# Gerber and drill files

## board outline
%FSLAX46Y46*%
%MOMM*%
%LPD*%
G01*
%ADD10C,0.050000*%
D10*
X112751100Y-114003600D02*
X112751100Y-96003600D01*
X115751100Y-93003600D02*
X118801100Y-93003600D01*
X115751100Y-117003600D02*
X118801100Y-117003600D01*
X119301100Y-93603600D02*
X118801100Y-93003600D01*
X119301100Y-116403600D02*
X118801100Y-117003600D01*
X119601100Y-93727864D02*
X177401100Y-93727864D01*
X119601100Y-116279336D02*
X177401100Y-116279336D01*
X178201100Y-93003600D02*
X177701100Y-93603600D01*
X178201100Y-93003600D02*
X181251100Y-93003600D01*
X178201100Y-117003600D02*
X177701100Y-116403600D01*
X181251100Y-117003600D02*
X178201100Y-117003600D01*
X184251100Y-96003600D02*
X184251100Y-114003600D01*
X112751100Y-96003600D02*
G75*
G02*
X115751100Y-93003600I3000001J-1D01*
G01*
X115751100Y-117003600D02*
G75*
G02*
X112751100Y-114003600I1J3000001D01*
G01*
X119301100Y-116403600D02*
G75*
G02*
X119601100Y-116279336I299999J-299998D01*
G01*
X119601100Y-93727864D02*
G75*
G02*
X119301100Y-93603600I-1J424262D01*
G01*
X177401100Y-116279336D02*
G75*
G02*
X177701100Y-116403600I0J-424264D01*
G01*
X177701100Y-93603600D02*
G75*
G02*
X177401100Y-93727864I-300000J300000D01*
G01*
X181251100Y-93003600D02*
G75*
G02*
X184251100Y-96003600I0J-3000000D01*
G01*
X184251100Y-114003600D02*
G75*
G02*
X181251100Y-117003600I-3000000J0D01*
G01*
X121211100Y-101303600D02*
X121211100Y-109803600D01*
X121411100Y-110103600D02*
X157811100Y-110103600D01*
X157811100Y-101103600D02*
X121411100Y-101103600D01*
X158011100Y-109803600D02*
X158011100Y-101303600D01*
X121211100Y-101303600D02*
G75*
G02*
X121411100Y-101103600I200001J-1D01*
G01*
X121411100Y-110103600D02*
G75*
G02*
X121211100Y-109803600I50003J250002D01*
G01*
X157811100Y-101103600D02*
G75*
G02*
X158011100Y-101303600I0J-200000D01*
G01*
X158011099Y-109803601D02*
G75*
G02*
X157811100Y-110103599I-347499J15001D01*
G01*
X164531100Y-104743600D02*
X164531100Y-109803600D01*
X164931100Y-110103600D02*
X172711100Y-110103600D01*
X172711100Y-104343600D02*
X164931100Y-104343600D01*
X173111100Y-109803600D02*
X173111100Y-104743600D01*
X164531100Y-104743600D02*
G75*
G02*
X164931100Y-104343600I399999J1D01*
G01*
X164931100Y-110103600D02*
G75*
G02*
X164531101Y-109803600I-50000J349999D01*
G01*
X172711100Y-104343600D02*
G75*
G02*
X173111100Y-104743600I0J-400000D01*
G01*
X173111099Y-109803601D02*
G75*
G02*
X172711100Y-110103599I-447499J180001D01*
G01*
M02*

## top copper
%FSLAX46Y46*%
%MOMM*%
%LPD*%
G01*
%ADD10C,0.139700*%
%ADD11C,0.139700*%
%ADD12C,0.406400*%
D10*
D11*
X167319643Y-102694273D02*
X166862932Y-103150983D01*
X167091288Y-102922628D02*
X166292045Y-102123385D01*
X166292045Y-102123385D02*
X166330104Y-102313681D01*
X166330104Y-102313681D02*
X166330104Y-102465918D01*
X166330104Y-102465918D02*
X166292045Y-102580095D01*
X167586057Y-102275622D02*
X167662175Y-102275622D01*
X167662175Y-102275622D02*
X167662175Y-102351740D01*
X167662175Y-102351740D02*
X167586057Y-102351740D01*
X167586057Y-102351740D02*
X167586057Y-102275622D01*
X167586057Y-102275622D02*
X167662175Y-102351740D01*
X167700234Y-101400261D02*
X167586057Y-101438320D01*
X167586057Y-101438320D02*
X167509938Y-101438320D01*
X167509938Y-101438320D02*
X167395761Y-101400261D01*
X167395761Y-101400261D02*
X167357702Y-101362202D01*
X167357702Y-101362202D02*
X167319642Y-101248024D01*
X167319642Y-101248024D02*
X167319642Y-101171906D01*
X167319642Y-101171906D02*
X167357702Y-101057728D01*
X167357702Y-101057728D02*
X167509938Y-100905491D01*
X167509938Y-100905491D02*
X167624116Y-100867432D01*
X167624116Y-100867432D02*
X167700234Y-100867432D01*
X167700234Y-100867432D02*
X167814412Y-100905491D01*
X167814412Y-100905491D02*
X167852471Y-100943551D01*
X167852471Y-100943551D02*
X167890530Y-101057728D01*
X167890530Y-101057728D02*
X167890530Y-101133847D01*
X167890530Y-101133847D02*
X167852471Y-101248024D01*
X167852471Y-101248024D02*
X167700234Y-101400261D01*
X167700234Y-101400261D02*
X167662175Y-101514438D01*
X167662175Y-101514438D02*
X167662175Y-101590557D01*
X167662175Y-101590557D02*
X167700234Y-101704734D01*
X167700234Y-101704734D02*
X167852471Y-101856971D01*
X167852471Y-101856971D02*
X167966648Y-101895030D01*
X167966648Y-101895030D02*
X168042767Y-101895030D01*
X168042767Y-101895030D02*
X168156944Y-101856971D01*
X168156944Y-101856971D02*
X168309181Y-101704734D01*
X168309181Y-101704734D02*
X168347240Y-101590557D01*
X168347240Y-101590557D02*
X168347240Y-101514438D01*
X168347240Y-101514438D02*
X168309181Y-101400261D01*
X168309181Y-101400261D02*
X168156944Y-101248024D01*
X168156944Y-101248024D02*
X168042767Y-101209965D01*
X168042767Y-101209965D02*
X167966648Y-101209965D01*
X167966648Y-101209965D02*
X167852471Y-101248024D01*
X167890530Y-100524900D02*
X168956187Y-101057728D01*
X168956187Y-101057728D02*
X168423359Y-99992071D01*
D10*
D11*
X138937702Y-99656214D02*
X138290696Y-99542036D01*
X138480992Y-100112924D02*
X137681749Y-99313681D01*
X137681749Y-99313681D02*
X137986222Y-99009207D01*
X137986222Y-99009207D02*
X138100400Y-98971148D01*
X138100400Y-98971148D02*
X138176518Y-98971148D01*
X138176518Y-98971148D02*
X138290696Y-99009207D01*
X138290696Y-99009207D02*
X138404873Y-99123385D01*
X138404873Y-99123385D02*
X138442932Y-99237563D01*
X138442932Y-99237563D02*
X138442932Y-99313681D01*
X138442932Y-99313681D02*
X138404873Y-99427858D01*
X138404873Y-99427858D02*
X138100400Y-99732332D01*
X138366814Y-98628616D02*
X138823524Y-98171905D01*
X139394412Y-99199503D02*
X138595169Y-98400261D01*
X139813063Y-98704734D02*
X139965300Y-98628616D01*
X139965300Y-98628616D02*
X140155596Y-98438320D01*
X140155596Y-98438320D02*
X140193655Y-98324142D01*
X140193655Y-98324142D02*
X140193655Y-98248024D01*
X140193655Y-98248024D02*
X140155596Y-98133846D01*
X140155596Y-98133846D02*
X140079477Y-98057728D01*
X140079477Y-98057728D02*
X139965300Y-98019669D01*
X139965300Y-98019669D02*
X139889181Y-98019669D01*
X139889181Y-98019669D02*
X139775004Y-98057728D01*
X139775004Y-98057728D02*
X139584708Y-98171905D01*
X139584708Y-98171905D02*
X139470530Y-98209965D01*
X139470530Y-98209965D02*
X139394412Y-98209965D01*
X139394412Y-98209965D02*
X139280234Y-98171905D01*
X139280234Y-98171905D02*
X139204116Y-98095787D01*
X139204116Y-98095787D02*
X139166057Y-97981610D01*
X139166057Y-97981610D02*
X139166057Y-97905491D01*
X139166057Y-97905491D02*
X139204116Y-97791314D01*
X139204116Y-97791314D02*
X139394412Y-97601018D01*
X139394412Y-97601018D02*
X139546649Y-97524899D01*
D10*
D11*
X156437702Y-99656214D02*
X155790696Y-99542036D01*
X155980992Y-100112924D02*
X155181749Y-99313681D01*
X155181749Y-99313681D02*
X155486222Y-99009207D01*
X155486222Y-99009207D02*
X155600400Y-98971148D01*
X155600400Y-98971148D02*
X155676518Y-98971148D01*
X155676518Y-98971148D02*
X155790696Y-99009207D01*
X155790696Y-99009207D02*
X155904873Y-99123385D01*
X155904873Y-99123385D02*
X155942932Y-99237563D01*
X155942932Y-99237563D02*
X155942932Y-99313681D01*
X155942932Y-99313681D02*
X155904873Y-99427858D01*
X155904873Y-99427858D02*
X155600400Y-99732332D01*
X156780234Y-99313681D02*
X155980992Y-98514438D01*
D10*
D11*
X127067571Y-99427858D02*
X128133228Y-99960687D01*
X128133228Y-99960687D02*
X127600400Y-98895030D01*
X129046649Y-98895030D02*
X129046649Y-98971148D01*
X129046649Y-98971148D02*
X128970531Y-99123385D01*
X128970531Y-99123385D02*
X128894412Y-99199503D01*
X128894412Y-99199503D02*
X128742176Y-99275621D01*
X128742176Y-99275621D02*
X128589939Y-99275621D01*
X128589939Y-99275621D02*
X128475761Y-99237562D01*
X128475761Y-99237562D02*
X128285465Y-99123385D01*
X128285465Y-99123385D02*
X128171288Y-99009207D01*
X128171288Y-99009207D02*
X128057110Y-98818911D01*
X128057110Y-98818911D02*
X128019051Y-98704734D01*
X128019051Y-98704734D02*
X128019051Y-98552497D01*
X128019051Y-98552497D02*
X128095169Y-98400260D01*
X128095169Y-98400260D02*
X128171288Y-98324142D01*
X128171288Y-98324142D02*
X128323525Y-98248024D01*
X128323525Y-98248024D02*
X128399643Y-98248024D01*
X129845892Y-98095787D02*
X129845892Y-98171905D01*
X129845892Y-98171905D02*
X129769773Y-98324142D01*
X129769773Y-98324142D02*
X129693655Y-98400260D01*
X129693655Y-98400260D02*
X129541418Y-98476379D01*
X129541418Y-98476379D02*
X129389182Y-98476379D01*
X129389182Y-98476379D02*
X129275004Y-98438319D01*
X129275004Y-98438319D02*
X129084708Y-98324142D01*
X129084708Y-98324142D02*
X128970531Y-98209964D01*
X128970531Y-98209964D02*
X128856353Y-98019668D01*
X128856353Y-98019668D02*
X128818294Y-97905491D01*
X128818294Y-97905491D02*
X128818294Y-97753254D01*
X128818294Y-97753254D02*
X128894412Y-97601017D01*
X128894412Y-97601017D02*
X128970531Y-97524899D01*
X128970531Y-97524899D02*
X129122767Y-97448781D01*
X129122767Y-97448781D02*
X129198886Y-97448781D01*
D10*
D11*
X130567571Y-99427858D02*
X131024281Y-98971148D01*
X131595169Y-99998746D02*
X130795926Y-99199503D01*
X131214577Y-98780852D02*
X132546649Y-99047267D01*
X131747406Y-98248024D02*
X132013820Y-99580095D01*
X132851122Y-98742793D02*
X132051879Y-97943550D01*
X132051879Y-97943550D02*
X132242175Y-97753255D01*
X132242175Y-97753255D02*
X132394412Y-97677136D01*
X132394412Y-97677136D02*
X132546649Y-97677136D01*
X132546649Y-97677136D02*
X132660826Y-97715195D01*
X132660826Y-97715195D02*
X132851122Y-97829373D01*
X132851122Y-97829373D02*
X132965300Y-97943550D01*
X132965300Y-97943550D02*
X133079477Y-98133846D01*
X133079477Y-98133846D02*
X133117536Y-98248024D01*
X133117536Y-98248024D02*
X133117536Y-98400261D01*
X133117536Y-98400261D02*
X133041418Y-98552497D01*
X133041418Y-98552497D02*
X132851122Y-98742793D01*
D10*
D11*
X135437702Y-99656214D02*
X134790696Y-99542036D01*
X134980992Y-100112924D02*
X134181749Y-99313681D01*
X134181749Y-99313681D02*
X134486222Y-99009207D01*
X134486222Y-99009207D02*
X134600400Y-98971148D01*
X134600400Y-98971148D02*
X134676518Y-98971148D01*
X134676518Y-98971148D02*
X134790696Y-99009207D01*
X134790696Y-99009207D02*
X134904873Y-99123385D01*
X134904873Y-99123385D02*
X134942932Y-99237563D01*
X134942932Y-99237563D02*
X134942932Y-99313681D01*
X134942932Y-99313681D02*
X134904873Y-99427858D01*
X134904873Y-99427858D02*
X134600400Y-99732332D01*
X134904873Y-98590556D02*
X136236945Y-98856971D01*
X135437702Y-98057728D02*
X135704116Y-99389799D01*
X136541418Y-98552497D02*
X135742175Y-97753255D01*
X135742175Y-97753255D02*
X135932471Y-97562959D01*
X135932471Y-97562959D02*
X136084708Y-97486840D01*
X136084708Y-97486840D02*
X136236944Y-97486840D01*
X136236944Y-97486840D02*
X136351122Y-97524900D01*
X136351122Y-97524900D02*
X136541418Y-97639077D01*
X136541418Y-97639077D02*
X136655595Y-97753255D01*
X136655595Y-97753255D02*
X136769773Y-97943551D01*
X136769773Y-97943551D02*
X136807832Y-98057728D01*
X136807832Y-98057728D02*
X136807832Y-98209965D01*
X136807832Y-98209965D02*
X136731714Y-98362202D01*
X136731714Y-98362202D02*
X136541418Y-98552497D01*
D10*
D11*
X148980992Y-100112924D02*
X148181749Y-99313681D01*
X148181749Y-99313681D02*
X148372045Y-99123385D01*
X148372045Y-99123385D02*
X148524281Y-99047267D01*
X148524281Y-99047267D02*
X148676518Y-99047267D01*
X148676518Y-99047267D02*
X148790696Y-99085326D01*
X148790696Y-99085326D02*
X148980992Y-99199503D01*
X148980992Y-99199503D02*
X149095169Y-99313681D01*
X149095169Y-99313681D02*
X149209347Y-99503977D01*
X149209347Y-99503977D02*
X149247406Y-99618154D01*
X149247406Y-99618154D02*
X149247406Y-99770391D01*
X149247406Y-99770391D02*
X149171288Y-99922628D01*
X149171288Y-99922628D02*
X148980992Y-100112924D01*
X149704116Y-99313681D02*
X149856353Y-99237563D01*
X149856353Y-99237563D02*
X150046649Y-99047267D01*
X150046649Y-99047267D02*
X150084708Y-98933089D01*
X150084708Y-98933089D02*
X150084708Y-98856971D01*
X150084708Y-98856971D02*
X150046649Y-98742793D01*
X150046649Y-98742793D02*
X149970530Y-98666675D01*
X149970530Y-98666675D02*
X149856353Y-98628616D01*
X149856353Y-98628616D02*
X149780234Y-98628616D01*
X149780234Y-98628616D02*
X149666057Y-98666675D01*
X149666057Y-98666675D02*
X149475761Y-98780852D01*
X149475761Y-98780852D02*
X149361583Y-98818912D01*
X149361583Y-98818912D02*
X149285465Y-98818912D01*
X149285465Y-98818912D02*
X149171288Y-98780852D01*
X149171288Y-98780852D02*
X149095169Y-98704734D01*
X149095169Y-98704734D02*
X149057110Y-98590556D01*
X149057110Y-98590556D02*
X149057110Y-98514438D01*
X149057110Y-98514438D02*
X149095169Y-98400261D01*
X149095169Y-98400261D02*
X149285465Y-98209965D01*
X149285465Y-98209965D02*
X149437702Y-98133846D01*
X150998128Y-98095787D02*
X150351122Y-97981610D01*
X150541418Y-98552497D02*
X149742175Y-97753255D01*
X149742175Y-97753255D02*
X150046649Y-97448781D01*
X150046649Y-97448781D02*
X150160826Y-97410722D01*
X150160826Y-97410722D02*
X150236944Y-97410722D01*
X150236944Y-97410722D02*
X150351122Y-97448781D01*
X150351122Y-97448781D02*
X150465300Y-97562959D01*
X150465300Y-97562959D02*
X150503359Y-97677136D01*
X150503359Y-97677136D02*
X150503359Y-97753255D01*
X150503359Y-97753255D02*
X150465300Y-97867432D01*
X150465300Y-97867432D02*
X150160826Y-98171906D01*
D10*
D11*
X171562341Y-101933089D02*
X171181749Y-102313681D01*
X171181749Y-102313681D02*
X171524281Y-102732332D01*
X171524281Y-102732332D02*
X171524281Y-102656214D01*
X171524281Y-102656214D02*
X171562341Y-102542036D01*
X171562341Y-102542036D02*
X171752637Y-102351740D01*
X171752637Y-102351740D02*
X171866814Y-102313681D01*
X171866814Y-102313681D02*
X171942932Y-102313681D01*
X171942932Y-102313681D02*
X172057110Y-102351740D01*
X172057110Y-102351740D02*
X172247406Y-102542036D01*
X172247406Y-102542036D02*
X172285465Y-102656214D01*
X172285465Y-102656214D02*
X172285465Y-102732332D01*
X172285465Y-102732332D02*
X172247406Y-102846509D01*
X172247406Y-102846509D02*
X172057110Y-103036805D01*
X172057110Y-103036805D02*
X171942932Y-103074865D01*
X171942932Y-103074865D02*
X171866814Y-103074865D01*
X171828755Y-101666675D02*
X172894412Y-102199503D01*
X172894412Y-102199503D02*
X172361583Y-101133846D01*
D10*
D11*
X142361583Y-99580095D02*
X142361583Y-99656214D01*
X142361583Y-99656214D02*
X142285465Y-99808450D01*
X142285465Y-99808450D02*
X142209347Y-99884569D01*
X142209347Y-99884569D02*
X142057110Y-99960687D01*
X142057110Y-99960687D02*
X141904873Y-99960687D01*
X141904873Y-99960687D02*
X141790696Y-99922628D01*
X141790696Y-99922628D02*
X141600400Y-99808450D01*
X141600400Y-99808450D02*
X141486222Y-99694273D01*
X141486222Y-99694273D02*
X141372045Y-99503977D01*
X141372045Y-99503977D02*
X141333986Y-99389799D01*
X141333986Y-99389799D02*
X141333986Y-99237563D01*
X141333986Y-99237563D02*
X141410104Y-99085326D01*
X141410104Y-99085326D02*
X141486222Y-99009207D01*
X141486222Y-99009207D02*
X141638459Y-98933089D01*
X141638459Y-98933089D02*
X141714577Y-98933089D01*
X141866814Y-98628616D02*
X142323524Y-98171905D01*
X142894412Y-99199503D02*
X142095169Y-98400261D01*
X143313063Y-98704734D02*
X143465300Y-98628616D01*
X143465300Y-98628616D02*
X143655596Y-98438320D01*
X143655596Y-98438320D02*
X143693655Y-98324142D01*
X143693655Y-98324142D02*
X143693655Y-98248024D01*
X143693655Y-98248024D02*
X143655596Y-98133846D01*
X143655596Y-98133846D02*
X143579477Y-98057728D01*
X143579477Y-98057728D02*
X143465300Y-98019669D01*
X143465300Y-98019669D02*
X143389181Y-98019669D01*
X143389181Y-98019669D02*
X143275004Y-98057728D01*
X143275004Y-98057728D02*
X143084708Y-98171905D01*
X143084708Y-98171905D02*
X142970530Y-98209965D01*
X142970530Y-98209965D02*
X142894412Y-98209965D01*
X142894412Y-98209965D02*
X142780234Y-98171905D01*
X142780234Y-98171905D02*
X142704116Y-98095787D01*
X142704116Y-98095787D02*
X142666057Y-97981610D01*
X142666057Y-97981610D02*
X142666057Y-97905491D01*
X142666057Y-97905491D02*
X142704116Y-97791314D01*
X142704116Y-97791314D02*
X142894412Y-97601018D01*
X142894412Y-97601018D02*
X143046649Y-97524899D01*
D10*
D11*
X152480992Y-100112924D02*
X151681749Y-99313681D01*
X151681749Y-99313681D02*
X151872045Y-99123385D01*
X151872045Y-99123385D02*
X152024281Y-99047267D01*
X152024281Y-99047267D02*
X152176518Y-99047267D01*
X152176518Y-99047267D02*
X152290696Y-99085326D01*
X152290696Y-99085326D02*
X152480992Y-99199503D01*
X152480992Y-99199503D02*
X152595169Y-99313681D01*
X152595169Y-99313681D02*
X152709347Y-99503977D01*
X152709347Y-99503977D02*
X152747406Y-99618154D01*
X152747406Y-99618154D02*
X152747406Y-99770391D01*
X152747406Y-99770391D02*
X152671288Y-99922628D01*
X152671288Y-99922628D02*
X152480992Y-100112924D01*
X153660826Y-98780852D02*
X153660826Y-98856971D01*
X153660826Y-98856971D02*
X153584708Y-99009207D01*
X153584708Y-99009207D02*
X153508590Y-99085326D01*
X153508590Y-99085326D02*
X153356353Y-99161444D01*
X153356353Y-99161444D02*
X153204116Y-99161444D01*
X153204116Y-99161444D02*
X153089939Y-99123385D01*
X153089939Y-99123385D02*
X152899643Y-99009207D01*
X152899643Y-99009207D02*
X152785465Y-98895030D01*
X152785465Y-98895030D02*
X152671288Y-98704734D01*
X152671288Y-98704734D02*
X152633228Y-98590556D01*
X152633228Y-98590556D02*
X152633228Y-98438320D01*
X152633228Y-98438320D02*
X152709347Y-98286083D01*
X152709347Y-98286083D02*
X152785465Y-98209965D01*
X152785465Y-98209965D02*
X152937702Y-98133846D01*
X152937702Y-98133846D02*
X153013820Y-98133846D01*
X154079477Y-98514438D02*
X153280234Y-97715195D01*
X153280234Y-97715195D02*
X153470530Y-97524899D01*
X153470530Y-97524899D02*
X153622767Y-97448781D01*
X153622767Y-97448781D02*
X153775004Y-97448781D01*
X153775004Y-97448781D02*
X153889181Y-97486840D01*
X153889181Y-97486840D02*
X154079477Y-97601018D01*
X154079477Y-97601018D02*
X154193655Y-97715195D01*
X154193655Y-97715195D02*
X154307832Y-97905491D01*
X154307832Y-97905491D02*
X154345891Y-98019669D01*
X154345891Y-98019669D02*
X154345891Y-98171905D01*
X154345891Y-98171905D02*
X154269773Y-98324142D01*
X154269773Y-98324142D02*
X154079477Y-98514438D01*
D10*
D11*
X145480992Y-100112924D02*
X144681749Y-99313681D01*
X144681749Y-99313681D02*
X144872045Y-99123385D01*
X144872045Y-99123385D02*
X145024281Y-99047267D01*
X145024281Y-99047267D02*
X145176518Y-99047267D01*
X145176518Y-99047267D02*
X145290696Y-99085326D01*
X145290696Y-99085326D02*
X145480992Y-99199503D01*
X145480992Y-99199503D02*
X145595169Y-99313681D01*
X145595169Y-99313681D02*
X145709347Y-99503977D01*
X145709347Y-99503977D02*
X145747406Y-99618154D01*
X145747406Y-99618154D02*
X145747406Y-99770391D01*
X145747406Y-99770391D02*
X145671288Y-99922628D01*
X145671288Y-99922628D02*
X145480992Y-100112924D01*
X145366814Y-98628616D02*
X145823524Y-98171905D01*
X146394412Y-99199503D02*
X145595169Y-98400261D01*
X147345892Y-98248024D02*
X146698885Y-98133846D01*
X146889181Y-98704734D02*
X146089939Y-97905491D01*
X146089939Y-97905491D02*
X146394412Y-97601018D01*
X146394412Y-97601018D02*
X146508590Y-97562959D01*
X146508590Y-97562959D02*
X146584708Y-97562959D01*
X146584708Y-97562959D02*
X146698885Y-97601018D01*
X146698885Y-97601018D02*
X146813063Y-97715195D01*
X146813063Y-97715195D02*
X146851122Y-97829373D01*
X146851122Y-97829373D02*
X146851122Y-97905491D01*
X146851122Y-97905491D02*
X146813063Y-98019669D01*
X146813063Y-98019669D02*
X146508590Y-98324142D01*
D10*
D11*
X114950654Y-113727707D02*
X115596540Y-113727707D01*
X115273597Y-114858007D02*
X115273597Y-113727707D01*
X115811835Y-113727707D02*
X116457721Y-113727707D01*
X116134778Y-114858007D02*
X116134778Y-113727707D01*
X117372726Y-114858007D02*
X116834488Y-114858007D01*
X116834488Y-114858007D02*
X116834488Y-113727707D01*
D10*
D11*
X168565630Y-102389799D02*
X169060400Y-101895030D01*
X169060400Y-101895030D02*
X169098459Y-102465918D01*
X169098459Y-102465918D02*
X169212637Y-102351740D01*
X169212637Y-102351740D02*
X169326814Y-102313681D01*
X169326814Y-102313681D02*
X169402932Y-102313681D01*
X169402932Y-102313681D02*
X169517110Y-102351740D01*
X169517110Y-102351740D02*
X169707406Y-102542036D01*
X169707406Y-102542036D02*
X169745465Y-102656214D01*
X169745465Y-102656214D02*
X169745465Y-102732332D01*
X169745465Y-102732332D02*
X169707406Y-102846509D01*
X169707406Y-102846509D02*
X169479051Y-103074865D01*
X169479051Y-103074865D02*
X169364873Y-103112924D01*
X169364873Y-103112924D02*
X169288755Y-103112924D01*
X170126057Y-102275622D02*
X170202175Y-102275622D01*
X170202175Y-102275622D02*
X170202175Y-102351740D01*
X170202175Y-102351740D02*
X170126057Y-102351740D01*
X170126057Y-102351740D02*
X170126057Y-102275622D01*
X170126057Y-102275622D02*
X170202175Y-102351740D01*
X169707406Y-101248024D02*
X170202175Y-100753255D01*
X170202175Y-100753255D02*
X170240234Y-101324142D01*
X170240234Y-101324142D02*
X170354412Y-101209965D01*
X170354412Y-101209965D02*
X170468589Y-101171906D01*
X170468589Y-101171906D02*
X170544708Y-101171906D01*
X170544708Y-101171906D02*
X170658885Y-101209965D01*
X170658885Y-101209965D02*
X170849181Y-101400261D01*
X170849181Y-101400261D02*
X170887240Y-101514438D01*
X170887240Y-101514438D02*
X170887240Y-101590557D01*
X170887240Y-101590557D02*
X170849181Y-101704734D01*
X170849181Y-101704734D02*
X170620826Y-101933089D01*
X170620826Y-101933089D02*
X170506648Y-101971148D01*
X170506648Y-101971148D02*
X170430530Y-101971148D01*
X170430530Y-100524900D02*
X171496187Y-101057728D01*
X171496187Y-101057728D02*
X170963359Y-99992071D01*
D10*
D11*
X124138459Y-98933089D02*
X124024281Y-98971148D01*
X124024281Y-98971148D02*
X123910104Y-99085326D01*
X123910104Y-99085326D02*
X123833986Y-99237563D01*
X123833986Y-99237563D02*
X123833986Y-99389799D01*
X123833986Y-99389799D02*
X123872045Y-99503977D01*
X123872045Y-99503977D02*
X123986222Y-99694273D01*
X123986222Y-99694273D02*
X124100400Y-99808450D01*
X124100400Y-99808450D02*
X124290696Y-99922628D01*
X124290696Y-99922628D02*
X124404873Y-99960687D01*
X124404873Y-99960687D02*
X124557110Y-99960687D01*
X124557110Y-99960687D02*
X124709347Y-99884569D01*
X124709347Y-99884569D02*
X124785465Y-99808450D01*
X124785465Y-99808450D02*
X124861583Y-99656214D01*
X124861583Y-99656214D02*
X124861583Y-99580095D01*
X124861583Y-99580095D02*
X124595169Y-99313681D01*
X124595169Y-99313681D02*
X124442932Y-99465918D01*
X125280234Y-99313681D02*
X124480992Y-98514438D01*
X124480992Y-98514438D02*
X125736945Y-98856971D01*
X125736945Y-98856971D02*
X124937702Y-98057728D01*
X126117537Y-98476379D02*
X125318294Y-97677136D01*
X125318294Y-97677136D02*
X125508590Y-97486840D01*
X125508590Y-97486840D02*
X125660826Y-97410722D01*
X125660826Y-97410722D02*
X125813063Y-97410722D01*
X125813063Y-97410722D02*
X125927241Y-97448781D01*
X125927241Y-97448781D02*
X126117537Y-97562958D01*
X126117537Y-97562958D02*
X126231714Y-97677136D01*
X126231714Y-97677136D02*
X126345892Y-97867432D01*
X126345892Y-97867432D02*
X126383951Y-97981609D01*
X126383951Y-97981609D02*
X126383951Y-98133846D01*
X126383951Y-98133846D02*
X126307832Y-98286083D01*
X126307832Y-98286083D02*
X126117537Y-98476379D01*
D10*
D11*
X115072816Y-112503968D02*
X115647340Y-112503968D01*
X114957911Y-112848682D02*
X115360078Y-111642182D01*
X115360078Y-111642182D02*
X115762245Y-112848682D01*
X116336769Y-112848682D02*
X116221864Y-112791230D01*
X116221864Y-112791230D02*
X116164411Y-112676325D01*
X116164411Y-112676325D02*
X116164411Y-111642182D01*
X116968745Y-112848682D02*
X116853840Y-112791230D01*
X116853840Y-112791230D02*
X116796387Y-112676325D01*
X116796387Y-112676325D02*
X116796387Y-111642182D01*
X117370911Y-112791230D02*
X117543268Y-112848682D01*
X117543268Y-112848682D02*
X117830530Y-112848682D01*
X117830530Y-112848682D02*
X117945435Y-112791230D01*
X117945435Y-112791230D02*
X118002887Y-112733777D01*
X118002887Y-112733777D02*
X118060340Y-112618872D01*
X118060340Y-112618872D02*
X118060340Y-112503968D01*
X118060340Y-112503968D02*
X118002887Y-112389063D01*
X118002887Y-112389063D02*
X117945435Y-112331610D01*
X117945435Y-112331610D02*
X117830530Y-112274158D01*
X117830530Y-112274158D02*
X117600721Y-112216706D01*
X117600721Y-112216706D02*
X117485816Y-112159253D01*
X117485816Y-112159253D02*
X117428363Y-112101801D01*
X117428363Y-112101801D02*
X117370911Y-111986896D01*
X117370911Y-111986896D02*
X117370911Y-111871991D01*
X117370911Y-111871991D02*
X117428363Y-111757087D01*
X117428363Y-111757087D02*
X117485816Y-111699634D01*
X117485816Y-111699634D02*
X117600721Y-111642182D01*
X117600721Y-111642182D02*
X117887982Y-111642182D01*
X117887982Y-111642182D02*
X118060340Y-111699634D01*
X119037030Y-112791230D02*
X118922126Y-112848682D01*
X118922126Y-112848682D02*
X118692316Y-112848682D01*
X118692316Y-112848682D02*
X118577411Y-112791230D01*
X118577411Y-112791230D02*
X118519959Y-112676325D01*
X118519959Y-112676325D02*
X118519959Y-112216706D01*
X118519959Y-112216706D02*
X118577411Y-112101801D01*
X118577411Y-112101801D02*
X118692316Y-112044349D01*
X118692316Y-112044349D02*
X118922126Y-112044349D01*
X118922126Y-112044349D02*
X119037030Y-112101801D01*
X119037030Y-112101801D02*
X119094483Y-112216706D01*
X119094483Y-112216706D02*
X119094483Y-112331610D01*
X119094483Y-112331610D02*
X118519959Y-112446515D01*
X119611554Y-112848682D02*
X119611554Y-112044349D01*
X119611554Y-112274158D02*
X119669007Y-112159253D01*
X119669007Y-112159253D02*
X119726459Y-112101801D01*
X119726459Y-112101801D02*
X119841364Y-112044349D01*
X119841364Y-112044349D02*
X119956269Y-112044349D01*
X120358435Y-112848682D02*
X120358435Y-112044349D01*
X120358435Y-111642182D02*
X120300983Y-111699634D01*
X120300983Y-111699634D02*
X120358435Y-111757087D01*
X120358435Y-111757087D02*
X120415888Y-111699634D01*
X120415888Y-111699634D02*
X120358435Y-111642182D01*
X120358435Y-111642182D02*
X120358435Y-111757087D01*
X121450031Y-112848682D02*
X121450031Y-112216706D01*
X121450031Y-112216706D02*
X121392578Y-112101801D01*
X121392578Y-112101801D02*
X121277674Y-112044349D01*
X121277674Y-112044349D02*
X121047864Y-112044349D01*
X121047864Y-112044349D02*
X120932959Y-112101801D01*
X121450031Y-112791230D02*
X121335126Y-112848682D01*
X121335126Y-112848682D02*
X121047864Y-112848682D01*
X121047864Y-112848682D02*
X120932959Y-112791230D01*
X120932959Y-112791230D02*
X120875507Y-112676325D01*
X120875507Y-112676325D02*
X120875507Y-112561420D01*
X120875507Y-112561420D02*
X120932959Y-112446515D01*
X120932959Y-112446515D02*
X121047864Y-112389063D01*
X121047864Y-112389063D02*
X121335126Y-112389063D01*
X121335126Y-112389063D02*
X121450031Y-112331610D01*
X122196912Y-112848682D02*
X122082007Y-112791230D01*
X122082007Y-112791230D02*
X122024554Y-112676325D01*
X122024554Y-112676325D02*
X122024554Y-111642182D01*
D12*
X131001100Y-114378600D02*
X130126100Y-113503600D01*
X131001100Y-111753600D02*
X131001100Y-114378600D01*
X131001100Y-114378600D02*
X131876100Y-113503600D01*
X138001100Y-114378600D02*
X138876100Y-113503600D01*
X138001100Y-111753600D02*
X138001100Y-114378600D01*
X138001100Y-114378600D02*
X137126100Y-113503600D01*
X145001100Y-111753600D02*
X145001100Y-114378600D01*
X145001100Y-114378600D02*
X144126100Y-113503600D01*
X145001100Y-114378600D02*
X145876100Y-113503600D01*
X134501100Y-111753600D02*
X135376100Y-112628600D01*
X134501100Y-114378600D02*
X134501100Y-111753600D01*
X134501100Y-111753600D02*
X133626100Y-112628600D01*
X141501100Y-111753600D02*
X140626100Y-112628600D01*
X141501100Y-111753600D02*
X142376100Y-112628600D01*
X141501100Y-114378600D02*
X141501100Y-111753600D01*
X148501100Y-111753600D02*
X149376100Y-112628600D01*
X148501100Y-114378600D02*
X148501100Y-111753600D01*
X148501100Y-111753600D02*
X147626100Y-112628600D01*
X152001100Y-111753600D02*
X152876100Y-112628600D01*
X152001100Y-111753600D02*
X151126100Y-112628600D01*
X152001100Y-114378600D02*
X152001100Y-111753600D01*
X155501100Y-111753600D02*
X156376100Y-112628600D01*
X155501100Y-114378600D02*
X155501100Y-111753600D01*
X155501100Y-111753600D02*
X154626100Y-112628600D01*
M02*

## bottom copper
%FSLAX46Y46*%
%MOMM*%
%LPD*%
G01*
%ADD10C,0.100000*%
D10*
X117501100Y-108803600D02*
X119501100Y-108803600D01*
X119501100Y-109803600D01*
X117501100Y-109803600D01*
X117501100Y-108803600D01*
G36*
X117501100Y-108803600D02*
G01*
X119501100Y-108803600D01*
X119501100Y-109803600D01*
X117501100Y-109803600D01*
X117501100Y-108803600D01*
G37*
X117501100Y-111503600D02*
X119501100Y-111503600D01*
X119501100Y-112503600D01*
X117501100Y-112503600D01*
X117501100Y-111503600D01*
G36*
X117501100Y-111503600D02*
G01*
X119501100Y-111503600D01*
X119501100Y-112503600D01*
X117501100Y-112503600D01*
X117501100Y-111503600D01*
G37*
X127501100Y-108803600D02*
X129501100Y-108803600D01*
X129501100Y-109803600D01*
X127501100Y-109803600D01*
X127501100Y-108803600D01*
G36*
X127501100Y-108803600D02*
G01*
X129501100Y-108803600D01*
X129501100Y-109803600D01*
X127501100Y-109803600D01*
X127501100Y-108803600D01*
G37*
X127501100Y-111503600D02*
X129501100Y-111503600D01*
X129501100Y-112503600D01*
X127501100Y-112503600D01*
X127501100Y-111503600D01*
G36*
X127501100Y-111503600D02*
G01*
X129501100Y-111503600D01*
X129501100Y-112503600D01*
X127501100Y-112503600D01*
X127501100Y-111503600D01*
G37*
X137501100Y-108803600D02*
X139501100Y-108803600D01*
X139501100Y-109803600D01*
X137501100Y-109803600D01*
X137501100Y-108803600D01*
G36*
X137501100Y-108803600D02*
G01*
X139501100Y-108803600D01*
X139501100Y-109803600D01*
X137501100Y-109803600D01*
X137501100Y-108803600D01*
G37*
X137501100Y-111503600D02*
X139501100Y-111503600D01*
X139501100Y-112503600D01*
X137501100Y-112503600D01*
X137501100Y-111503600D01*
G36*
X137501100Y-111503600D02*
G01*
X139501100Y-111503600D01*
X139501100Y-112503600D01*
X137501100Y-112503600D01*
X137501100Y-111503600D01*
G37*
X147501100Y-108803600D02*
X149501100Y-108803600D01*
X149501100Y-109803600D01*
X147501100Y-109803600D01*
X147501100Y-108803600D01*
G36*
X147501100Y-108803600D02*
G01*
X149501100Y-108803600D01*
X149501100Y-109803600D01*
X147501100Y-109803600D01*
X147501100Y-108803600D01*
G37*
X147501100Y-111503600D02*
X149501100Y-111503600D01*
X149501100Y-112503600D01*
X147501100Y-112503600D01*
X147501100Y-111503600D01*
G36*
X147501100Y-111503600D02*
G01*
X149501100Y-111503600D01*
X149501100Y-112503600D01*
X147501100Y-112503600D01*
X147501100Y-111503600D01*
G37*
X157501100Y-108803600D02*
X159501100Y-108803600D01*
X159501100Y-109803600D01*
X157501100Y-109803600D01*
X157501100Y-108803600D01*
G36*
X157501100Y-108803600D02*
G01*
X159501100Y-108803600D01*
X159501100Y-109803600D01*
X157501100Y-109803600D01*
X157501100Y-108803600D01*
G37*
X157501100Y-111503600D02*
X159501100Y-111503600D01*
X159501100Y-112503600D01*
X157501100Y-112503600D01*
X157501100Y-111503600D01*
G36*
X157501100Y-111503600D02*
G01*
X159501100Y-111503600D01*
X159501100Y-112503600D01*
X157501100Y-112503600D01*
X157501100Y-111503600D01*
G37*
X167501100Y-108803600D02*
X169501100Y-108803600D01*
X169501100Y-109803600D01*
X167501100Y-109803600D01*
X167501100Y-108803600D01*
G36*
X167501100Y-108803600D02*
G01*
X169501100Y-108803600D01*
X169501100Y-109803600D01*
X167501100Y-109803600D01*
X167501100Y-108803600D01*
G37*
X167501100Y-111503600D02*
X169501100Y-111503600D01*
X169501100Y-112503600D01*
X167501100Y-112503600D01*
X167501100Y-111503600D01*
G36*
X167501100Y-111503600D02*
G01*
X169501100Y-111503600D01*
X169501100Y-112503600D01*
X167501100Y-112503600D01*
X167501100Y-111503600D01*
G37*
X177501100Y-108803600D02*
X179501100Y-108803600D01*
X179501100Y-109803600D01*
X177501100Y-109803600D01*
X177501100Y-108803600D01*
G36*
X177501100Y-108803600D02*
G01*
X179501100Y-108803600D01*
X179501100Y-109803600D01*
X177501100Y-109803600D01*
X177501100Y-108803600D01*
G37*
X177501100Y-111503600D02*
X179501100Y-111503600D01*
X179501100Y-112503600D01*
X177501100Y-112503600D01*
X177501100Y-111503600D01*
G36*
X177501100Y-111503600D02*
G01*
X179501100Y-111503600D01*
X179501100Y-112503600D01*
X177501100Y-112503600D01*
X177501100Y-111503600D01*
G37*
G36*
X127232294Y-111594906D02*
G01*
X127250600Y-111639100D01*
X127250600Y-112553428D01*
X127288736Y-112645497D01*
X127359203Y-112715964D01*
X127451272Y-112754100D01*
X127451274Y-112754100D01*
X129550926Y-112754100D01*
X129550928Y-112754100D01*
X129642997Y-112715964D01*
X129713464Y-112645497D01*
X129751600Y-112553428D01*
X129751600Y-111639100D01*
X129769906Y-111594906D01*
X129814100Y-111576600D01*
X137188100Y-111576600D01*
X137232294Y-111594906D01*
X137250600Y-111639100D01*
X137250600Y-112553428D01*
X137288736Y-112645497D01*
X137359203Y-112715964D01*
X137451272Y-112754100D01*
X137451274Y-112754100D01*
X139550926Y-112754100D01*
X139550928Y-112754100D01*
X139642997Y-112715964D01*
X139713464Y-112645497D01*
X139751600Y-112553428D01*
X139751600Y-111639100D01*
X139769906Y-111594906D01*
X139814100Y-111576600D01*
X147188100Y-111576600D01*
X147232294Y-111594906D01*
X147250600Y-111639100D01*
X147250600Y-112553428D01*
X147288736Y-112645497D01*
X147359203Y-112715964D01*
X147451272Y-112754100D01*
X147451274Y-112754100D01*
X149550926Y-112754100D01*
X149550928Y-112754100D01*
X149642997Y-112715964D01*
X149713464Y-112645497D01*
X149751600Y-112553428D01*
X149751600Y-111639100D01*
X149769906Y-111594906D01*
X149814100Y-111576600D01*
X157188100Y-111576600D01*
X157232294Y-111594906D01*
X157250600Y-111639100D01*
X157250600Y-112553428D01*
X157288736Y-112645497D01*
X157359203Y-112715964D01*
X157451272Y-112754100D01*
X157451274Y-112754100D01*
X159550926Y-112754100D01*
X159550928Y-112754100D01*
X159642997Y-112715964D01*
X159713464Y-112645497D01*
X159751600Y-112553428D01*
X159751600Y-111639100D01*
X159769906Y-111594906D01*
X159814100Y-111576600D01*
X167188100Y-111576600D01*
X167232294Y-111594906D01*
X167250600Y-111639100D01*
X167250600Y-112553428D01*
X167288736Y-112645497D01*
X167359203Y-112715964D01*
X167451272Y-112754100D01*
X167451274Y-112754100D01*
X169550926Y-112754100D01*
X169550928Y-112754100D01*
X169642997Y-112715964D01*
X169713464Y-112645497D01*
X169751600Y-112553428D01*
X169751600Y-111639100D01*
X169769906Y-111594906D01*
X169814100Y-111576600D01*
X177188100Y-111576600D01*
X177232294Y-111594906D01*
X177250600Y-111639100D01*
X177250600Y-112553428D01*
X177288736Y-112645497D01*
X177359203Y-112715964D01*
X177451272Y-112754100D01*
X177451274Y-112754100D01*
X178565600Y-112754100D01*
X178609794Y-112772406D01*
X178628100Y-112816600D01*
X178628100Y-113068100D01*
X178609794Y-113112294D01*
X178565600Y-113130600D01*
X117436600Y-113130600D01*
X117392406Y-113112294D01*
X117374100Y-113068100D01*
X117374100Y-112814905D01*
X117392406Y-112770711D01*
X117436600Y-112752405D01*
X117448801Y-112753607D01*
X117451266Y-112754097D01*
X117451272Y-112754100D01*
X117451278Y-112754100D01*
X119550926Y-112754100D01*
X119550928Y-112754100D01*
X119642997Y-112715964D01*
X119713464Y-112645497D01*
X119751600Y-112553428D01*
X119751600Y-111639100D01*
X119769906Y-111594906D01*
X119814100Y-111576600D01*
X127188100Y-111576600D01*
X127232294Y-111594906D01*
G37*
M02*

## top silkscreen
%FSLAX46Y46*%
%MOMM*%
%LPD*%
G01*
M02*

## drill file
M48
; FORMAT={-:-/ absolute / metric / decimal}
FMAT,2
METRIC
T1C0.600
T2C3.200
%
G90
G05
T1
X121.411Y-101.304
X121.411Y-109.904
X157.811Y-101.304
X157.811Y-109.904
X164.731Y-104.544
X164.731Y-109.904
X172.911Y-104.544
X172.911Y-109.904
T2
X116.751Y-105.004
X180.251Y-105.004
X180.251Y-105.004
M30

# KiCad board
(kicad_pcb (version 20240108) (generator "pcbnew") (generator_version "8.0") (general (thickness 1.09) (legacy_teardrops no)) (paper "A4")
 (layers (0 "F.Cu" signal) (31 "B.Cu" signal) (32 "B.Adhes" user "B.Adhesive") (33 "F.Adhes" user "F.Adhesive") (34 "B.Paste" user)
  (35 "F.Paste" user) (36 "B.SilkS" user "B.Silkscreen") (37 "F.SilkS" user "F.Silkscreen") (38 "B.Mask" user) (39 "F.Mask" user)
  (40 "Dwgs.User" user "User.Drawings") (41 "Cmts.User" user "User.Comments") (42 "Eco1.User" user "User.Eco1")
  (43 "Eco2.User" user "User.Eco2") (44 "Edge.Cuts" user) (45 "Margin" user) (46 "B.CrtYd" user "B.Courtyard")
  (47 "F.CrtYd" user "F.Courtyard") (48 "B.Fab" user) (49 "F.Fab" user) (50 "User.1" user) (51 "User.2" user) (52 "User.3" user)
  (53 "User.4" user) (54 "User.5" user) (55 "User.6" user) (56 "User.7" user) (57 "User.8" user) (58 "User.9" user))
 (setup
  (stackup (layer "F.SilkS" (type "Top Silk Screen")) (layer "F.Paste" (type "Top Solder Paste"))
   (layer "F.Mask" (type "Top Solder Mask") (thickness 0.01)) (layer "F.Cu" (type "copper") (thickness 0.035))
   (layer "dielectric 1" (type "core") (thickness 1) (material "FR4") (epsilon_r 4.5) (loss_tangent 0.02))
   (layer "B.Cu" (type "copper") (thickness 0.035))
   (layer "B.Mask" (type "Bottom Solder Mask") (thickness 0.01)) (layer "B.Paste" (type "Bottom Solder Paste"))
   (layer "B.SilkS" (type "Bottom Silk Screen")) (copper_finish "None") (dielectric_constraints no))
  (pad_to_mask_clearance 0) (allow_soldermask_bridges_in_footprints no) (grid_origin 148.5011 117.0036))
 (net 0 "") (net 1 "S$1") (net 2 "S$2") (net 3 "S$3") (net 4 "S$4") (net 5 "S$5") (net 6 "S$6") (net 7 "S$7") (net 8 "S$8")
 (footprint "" (layer "F.Cu") (at 180.2511 105.0036)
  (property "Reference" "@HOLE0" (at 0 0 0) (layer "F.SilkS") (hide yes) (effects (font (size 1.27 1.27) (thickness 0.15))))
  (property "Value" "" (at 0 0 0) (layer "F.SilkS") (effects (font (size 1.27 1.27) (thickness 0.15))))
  (pad "" np_thru_hole circle (at 0 0) (size 3.2 3.2) (drill 3.2) (layers "*.Cu" "*.Mask")))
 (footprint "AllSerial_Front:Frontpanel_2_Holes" (layer "F.Cu") (at 148.5011 117.0036)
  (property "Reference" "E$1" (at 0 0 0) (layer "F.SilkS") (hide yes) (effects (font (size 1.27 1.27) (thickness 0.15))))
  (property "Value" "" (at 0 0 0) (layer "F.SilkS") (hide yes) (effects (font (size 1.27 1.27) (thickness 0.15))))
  (fp_rect (start -31 -8.2) (end -29 -7.2) (stroke (width 0.1) (type solid)) (fill solid) (layer "B.Cu"))
  (fp_rect (start -31 -5.5) (end -29 -4.5) (stroke (width 0.1) (type solid)) (fill solid) (layer "B.Cu"))
  (fp_rect (start -21 -8.2) (end -19 -7.2) (stroke (width 0.1) (type solid)) (fill solid) (layer "B.Cu"))
  (fp_rect (start -21 -5.5) (end -19 -4.5) (stroke (width 0.1) (type solid)) (fill solid) (layer "B.Cu"))
  (fp_rect (start -11 -8.2) (end -9 -7.2) (stroke (width 0.1) (type solid)) (fill solid) (layer "B.Cu"))
  (fp_rect (start -11 -5.5) (end -9 -4.5) (stroke (width 0.1) (type solid)) (fill solid) (layer "B.Cu"))
  (fp_rect (start -1 -8.2) (end 1 -7.2) (stroke (width 0.1) (type solid)) (fill solid) (layer "B.Cu"))
  (fp_rect (start -1 -5.5) (end 1 -4.5) (stroke (width 0.1) (type solid)) (fill solid) (layer "B.Cu"))
  (fp_rect (start 9 -8.2) (end 11 -7.2) (stroke (width 0.1) (type solid)) (fill solid) (layer "B.Cu"))
  (fp_rect (start 9 -5.5) (end 11 -4.5) (stroke (width 0.1) (type solid)) (fill solid) (layer "B.Cu"))
  (fp_rect (start 19 -8.2) (end 21 -7.2) (stroke (width 0.1) (type solid)) (fill solid) (layer "B.Cu"))
  (fp_rect (start 19 -5.5) (end 21 -4.5) (stroke (width 0.1) (type solid)) (fill solid) (layer "B.Cu"))
  (fp_rect (start 29 -8.2) (end 31 -7.2) (stroke (width 0.1) (type solid)) (fill solid) (layer "B.Cu"))
  (fp_rect (start 29 -5.5) (end 31 -4.5) (stroke (width 0.1) (type solid)) (fill solid) (layer "B.Cu"))
  (fp_line (start -35.75 -3) (end -35.75 -21) (stroke (width 0.05) (type solid)) (layer "Edge.Cuts"))
  (fp_line (start -32.75 -24) (end -29.7 -24) (stroke (width 0.05) (type solid)) (layer "Edge.Cuts"))
  (fp_line (start -32.75 0) (end -29.7 0) (stroke (width 0.05) (type default)) (layer "Edge.Cuts"))
  (fp_line (start -29.2 -23.4) (end -29.7 -24) (stroke (width 0.05) (type default)) (layer "Edge.Cuts"))
  (fp_line (start -29.2 -0.6) (end -29.7 0) (stroke (width 0.05) (type default)) (layer "Edge.Cuts"))
  (fp_line (start -28.9 -23.275736) (end 28.9 -23.275736) (stroke (width 0.05) (type default)) (layer "Edge.Cuts"))
  (fp_line (start -28.9 -0.724264) (end 28.9 -0.724264) (stroke (width 0.05) (type default)) (layer "Edge.Cuts"))
  (fp_line (start 29.7 -24) (end 29.2 -23.4) (stroke (width 0.05) (type default)) (layer "Edge.Cuts"))
  (fp_line (start 29.7 -24) (end 32.75 -24) (stroke (width 0.05) (type solid)) (layer "Edge.Cuts"))
  (fp_line (start 29.7 0) (end 29.2 -0.6) (stroke (width 0.05) (type default)) (layer "Edge.Cuts"))
  (fp_line (start 32.75 0) (end 29.7 0) (stroke (width 0.05) (type default)) (layer "Edge.Cuts"))
  (fp_line (start 35.75 -21) (end 35.75 -3) (stroke (width 0.05) (type solid)) (layer "Edge.Cuts"))
  (fp_arc (start -35.75 -21) (mid -34.87132 -23.12132) (end -32.75 -24) (stroke (width 0.05) (type solid)) (layer "Edge.Cuts"))
  (fp_arc (start -32.75 0) (mid -34.87132 -0.87868) (end -35.75 -3) (stroke (width 0.05) (type solid)) (layer "Edge.Cuts"))
  (fp_arc (start -29.2 -0.6) (mid -29.062359 -0.691969) (end -28.9 -0.724264) (stroke (width 0.05) (type default)) (layer "Edge.Cuts"))
  (fp_arc (start -28.9 -23.275736) (mid -29.062359 -23.308031) (end -29.2 -23.4) (stroke (width 0.05) (type default)) (layer "Edge.Cuts"))
  (fp_arc (start 28.9 -0.724264) (mid 29.062359 -0.691969) (end 29.2 -0.6) (stroke (width 0.05) (type default)) (layer "Edge.Cuts"))
  (fp_arc (start 29.2 -23.4) (mid 29.062359 -23.308031) (end 28.9 -23.275736) (stroke (width 0.05) (type default)) (layer "Edge.Cuts"))
  (fp_arc (start 32.75 -24) (mid 34.87132 -23.12132) (end 35.75 -21) (stroke (width 0.05) (type solid)) (layer "Edge.Cuts"))
  (fp_arc (start 35.75 -3) (mid 34.87132 -0.87868) (end 32.75 0) (stroke (width 0.05) (type solid)) (layer "Edge.Cuts"))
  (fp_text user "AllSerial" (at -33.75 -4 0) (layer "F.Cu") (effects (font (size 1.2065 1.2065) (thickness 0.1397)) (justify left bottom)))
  (pad "" np_thru_hole circle (at -31.75 -12) (size 3.2 3.2) (drill 3.2) (layers "*.Cu" "*.Mask"))
  (pad "" np_thru_hole circle (at 31.75 -12) (size 3.2 3.2) (drill 3.2) (layers "*.Cu" "*.Mask")))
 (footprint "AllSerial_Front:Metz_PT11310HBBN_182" (layer "F.Cu") (at 139.6111 117.0036)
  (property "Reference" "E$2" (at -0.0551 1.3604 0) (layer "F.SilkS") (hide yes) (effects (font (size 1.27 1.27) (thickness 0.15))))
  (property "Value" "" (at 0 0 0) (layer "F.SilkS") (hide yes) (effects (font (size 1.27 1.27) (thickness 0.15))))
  (fp_line (start -18.4 -15.7) (end -18.4 -7.2) (stroke (width 0.05) (type solid)) (layer "Edge.Cuts"))
  (fp_line (start -18.2 -6.9) (end 18.2 -6.9) (stroke (width 0.05) (type solid)) (layer "Edge.Cuts"))
  (fp_line (start 18.2 -15.9) (end -18.2 -15.9) (stroke (width 0.05) (type solid)) (layer "Edge.Cuts"))
  (fp_line (start 18.4 -7.2) (end 18.4 -15.7) (stroke (width 0.05) (type solid)) (layer "Edge.Cuts"))
  (fp_arc (start -18.4 -15.7) (mid -18.341421 -15.841421) (end -18.2 -15.9) (stroke (width 0.05) (type solid)) (layer "Edge.Cuts"))
  (fp_arc (start -18.2 -6.9) (mid -18.362131 -7.008579) (end -18.4 -7.2) (stroke (width 0.05) (type solid)) (layer "Edge.Cuts"))
  (fp_arc (start 18.2 -15.9) (mid 18.341421 -15.841421) (end 18.4 -15.7) (stroke (width 0.05) (type solid)) (layer "Edge.Cuts"))
  (fp_arc (start 18.399999 -7.199999) (mid 18.341906 -7.022062) (end 18.2 -6.9) (stroke (width 0.05) (type solid)) (layer "Edge.Cuts"))
  (pad "" np_thru_hole circle (at -18.2 -15.7) (size 0.6 0.6) (drill 0.6) (layers "*.Cu" "*.Mask"))
  (pad "" np_thru_hole circle (at -18.2 -7.1) (size 0.6 0.6) (drill 0.6) (layers "*.Cu" "*.Mask"))
  (pad "" np_thru_hole circle (at 18.2 -15.7) (size 0.6 0.6) (drill 0.6) (layers "*.Cu" "*.Mask"))
  (pad "" np_thru_hole circle (at 18.2 -7.1) (size 0.6 0.6) (drill 0.6) (layers "*.Cu" "*.Mask")))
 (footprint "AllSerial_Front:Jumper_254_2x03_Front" (layer "F.Cu") (at 168.8211 117.0036)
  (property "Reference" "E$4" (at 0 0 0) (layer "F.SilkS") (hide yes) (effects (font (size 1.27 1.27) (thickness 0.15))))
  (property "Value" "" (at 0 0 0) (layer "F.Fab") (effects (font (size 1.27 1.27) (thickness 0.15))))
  (fp_line (start -4.29 -12.26) (end -4.29 -7.2) (stroke (width 0.05) (type solid)) (layer "Edge.Cuts"))
  (fp_line (start -3.89 -6.9) (end 3.89 -6.9) (stroke (width 0.05) (type solid)) (layer "Edge.Cuts"))
  (fp_line (start 3.89 -12.66) (end -3.89 -12.66) (stroke (width 0.05) (type solid)) (layer "Edge.Cuts"))
  (fp_line (start 4.29 -7.2) (end 4.29 -12.26) (stroke (width 0.05) (type solid)) (layer "Edge.Cuts"))
  (fp_arc (start -4.29 -12.26) (mid -4.172843 -12.542843) (end -3.89 -12.66) (stroke (width 0.05) (type solid)) (layer "Edge.Cuts"))
  (fp_arc (start -3.89 -6.9) (mid -4.152132 -6.967157) (end -4.29 -7.2) (stroke (width 0.05) (type solid)) (layer "Edge.Cuts"))
  (fp_arc (start 3.89 -12.66) (mid 4.172843 -12.542843) (end 4.29 -12.26) (stroke (width 0.05) (type solid)) (layer "Edge.Cuts"))
  (fp_arc (start 4.289999 -7.199999) (mid 4.131906 -6.994124) (end 3.89 -6.9) (stroke (width 0.05) (type solid)) (layer "Edge.Cuts"))
  (pad "" np_thru_hole circle (at -4.09 -12.46) (size 0.6 0.6) (drill 0.6) (layers "*.Cu" "*.Mask"))
  (pad "" np_thru_hole circle (at -4.09 -7.1) (size 0.6 0.6) (drill 0.6) (layers "*.Cu" "*.Mask"))
  (pad "" np_thru_hole circle (at 4.09 -12.46) (size 0.6 0.6) (drill 0.6) (layers "*.Cu" "*.Mask"))
  (pad "" np_thru_hole circle (at 4.09 -7.1) (size 0.6 0.6) (drill 0.6) (layers "*.Cu" "*.Mask"))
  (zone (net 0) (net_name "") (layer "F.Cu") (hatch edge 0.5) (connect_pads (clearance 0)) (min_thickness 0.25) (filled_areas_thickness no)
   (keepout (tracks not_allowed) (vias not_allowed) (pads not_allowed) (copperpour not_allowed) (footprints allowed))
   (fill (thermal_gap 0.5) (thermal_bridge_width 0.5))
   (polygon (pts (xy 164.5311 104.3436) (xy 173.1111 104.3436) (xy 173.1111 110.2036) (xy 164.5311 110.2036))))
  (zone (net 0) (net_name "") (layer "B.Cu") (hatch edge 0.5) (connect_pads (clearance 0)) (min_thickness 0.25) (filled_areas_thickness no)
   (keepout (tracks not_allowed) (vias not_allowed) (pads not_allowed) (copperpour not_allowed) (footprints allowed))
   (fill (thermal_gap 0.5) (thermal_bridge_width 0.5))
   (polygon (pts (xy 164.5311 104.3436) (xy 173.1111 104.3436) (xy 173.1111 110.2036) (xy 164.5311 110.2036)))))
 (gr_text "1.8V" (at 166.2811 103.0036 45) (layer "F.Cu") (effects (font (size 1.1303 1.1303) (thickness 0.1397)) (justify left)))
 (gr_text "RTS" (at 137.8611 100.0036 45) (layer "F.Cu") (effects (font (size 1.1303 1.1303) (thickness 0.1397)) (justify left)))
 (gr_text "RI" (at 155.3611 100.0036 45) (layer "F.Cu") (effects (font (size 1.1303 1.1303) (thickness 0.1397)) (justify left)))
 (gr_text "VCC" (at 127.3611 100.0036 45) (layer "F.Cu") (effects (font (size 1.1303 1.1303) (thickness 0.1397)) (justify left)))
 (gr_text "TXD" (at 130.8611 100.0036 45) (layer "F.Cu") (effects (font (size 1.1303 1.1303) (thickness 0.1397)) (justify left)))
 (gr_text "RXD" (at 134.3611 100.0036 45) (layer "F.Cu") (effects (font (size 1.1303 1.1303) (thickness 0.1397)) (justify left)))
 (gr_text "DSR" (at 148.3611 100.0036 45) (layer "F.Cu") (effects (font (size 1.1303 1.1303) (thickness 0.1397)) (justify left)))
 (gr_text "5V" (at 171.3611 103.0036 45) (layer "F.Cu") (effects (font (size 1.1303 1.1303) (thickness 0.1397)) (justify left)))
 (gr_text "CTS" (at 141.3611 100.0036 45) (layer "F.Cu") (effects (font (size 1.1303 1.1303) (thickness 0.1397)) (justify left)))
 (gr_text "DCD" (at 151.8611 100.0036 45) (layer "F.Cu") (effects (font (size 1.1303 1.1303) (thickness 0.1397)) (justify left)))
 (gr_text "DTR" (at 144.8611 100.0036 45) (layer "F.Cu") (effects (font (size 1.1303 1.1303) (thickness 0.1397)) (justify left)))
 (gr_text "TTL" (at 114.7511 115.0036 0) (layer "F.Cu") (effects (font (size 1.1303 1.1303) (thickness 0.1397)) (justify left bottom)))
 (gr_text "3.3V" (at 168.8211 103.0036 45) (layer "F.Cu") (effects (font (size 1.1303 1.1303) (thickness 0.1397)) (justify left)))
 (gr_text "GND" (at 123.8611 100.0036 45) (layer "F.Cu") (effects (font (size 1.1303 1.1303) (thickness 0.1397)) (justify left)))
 (segment (start 131.0011 114.3786) (end 130.1261 113.5036) (width 0.4064) (layer "F.Cu") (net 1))
 (segment (start 131.0011 111.7536) (end 131.0011 114.3786) (width 0.4064) (layer "F.Cu") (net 1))
 (segment (start 131.0011 114.3786) (end 131.8761 113.5036) (width 0.4064) (layer "F.Cu") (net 1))
 (segment (start 138.0011 114.3786) (end 138.8761 113.5036) (width 0.4064) (layer "F.Cu") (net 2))
 (segment (start 138.0011 111.7536) (end 138.0011 114.3786) (width 0.4064) (layer "F.Cu") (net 2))
 (segment (start 138.0011 114.3786) (end 137.1261 113.5036) (width 0.4064) (layer "F.Cu") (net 2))
 (segment (start 145.0011 111.7536) (end 145.0011 114.3786) (width 0.4064) (layer "F.Cu") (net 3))
 (segment (start 145.0011 114.3786) (end 144.1261 113.5036) (width 0.4064) (layer "F.Cu") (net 3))
 (segment (start 145.0011 114.3786) (end 145.8761 113.5036) (width 0.4064) (layer "F.Cu") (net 3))
 (segment (start 134.5011 111.7536) (end 135.3761 112.6286) (width 0.4064) (layer "F.Cu") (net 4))
 (segment (start 134.5011 114.3786) (end 134.5011 111.7536) (width 0.4064) (layer "F.Cu") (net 4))
 (segment (start 134.5011 111.7536) (end 133.6261 112.6286) (width 0.4064) (layer "F.Cu") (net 4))
 (segment (start 141.5011 111.7536) (end 140.6261 112.6286) (width 0.4064) (layer "F.Cu") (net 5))
 (segment (start 141.5011 111.7536) (end 142.3761 112.6286) (width 0.4064) (layer "F.Cu") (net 5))
 (segment (start 141.5011 114.3786) (end 141.5011 111.7536) (width 0.4064) (layer "F.Cu") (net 5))
 (segment (start 148.5011 111.7536) (end 149.3761 112.6286) (width 0.4064) (layer "F.Cu") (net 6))
 (segment (start 148.5011 114.3786) (end 148.5011 111.7536) (width 0.4064) (layer "F.Cu") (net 6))
 (segment (start 148.5011 111.7536) (end 147.6261 112.6286) (width 0.4064) (layer "F.Cu") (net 6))
 (segment (start 152.0011 111.7536) (end 152.8761 112.6286) (width 0.4064) (layer "F.Cu") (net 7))
 (segment (start 152.0011 111.7536) (end 151.1261 112.6286) (width 0.4064) (layer "F.Cu") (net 7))
 (segment (start 152.0011 114.3786) (end 152.0011 111.7536) (width 0.4064) (layer "F.Cu") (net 7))
 (segment (start 155.5011 111.7536) (end 156.3761 112.6286) (width 0.4064) (layer "F.Cu") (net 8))
 (segment (start 155.5011 114.3786) (end 155.5011 111.7536) (width 0.4064) (layer "F.Cu") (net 8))
 (segment (start 155.5011 111.7536) (end 154.6261 112.6286) (width 0.4064) (layer "F.Cu") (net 8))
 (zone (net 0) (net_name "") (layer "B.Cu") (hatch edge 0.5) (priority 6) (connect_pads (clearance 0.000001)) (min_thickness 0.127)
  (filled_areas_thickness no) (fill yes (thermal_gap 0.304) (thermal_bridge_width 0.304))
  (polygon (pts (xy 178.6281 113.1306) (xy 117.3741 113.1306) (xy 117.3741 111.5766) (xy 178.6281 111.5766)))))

